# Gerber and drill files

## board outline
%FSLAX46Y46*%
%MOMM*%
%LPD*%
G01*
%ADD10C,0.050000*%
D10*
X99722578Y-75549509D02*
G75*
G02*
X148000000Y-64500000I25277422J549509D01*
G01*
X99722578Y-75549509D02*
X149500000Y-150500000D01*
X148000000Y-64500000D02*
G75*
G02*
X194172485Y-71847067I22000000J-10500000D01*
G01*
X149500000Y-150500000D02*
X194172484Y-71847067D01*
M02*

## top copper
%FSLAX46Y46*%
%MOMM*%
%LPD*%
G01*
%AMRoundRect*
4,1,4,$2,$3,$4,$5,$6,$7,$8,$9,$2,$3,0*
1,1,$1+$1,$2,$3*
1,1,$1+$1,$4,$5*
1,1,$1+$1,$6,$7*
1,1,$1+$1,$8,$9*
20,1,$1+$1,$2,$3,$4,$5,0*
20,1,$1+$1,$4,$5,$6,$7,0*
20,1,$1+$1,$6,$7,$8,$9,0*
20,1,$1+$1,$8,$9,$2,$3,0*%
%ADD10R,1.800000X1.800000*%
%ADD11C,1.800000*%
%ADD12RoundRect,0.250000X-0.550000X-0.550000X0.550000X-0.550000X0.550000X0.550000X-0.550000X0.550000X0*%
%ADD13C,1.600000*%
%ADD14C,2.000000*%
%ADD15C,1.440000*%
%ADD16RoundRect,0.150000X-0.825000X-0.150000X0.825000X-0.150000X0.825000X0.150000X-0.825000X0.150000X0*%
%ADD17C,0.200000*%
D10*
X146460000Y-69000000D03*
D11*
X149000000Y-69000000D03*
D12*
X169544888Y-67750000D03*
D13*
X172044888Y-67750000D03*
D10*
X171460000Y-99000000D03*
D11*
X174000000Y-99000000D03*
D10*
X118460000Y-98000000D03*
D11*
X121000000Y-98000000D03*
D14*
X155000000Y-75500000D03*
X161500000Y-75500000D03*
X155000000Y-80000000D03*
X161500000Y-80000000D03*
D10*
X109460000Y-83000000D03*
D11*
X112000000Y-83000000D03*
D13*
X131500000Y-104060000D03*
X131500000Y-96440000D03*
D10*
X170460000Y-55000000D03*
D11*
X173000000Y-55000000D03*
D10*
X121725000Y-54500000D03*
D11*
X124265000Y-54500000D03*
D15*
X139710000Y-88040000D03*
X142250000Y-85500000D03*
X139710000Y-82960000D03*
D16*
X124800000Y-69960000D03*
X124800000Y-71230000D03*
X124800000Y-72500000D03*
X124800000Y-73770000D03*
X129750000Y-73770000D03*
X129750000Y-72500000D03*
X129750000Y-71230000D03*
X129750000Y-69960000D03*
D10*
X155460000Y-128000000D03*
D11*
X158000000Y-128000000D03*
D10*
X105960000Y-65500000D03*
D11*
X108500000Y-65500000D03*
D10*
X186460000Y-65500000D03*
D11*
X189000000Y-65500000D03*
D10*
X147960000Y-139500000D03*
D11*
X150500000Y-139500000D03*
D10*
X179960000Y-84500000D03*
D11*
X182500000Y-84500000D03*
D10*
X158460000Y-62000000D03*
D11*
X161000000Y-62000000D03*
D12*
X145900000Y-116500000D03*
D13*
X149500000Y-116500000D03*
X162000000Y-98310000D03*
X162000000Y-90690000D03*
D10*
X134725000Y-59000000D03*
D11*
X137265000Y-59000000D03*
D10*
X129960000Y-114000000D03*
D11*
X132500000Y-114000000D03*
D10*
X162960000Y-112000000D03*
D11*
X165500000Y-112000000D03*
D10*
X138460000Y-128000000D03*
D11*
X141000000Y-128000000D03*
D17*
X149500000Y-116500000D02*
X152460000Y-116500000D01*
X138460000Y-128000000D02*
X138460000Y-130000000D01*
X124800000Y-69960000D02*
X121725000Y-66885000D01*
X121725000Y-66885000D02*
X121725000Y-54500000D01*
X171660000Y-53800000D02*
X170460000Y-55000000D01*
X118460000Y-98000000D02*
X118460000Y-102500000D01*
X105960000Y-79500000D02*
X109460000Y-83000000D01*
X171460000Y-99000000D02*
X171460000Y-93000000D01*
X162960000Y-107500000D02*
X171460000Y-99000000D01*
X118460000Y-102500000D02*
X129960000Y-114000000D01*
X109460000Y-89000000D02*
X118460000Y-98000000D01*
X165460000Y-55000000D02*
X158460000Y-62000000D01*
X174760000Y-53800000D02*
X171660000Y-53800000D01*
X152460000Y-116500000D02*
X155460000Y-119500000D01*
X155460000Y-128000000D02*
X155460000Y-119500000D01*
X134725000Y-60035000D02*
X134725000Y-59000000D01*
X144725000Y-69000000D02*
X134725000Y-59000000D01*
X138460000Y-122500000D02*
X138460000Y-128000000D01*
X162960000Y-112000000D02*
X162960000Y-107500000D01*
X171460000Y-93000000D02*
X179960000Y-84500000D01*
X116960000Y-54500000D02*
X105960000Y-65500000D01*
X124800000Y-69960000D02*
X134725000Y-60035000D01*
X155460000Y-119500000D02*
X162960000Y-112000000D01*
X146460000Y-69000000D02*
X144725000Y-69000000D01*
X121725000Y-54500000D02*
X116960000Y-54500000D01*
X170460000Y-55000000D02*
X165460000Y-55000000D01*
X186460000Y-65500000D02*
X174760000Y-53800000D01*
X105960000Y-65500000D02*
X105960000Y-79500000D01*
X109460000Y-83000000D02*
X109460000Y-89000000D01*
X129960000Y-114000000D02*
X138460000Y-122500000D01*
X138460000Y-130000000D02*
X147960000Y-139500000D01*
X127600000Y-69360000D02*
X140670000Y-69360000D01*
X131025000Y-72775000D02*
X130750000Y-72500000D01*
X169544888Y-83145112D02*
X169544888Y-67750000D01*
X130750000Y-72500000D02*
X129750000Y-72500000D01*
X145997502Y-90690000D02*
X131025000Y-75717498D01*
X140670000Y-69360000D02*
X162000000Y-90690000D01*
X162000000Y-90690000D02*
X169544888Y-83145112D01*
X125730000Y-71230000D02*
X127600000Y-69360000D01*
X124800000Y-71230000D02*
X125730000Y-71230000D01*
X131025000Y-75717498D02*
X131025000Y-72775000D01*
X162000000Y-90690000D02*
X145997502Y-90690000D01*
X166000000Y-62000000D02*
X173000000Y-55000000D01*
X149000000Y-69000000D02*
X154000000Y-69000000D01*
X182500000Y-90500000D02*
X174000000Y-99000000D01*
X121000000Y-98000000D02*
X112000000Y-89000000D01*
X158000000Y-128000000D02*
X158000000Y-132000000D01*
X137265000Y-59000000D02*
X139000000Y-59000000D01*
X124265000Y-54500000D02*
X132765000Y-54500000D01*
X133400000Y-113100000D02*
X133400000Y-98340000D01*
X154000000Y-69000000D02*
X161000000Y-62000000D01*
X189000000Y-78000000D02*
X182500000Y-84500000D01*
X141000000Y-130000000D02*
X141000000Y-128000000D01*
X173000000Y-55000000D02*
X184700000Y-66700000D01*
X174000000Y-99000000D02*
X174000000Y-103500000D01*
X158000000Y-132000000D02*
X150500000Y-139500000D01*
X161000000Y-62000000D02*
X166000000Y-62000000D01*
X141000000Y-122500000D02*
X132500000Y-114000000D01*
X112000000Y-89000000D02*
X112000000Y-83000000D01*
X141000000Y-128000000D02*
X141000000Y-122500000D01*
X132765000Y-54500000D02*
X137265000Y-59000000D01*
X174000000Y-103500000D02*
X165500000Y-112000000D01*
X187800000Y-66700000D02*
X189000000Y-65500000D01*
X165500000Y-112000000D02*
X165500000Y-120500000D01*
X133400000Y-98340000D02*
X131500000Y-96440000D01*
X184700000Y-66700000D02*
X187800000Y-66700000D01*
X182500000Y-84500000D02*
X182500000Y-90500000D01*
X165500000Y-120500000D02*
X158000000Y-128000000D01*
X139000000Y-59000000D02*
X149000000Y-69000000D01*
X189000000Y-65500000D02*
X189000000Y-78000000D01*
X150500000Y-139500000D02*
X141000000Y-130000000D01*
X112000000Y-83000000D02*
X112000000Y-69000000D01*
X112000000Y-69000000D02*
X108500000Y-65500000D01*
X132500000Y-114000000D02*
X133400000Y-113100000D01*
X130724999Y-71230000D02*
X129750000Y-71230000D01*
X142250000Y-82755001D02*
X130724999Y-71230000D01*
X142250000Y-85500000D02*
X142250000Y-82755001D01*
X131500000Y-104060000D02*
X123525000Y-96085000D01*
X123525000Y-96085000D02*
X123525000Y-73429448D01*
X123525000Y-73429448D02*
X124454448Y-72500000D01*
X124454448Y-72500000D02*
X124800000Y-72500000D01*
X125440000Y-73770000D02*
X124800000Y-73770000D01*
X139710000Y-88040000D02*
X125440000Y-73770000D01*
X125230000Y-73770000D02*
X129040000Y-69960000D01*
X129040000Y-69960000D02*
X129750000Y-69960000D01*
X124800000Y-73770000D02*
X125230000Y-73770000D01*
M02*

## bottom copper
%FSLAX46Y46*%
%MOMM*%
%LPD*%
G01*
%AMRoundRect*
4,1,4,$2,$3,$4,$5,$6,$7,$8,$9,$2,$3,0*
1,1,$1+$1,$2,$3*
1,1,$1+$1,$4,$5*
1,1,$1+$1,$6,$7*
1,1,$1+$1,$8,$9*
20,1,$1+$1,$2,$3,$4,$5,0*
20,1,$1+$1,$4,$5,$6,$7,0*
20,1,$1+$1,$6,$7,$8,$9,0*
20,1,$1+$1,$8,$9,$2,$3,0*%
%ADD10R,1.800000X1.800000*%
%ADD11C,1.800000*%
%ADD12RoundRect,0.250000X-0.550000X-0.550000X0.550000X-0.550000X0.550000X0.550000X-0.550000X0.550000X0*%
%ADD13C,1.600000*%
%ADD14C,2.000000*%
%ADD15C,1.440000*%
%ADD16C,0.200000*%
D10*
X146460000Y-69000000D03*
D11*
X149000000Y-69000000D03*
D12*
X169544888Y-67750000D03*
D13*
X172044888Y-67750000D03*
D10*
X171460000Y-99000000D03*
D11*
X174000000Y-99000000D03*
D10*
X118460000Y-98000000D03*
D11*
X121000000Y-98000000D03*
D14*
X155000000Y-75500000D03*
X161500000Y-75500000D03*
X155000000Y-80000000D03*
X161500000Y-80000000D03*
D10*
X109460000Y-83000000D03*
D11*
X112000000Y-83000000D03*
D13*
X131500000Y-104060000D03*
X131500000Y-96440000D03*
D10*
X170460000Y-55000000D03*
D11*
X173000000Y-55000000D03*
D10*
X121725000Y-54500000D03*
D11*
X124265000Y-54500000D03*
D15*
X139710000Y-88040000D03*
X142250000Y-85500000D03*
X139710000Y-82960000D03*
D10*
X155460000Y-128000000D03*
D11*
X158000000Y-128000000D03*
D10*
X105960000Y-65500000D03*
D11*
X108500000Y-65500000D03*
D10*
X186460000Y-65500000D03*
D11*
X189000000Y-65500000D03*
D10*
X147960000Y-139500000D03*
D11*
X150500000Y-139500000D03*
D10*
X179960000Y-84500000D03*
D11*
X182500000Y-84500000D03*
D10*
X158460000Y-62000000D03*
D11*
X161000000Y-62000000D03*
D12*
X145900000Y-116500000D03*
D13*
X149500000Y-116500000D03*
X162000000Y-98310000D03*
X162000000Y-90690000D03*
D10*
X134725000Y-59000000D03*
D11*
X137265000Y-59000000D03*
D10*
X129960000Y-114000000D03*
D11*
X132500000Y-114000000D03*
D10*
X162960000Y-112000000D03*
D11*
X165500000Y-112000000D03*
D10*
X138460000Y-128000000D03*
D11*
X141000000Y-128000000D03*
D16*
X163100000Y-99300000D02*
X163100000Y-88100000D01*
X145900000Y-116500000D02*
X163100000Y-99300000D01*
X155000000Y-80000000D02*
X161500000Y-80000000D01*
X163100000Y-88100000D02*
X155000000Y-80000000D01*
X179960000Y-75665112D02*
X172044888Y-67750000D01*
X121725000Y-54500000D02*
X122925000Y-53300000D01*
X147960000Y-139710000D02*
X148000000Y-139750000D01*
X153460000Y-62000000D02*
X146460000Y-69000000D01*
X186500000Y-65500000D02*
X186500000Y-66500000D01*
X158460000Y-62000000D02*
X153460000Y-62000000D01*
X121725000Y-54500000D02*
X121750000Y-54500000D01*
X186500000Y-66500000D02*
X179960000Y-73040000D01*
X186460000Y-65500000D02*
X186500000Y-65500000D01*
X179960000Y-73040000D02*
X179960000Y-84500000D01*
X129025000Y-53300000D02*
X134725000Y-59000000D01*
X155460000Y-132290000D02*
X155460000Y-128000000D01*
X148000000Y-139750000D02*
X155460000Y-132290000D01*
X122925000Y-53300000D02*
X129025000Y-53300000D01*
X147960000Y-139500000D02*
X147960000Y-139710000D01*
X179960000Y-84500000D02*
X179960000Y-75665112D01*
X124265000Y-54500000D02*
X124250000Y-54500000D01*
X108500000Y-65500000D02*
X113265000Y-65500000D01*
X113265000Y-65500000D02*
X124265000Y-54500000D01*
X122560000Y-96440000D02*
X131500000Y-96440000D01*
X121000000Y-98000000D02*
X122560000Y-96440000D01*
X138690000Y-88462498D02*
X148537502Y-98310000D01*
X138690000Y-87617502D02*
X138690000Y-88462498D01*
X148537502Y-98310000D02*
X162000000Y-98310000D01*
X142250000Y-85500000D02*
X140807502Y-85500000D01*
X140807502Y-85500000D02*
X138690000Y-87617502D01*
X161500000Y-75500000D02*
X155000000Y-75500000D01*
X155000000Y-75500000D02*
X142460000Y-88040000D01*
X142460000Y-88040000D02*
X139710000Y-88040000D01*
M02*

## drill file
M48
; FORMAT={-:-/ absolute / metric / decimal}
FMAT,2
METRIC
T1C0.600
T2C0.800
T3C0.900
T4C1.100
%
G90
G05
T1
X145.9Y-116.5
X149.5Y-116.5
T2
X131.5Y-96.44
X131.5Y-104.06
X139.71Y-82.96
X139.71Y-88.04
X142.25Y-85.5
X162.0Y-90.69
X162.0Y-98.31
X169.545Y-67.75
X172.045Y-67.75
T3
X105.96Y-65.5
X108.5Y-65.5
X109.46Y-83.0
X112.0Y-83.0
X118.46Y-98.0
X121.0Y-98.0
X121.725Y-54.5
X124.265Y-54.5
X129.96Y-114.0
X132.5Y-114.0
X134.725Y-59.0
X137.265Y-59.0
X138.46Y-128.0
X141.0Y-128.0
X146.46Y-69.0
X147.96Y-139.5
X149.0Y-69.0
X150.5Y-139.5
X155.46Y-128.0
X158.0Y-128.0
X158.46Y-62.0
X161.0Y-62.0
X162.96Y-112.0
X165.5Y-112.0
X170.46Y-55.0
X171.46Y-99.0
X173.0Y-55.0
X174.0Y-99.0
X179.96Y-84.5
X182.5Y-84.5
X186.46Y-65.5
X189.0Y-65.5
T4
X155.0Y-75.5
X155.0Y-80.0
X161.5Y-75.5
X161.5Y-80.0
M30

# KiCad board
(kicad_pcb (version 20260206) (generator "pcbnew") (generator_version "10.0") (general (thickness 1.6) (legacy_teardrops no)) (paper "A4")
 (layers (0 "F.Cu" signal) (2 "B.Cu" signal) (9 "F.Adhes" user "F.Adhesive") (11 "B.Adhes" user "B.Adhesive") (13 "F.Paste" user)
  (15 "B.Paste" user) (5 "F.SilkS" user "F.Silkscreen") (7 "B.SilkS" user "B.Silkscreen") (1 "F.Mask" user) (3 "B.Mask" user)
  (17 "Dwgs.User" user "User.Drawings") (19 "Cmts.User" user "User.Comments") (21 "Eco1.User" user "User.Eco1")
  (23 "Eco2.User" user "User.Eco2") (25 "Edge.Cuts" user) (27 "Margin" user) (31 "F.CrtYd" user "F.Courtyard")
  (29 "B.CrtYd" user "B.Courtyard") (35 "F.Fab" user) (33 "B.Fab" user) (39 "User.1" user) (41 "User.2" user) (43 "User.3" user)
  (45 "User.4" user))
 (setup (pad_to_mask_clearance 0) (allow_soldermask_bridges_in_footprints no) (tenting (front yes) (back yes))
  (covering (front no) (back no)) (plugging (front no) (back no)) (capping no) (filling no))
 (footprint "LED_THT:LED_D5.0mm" (layer "F.Cu") (at 146.46 69)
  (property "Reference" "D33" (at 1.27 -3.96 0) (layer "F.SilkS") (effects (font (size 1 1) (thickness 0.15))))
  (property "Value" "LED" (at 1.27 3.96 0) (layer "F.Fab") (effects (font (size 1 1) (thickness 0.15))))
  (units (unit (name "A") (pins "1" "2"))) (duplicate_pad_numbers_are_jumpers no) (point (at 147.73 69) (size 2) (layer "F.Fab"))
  (pad "1" thru_hole rect (at 0 0) (size 1.8 1.8) (drill 0.9) (layers "*.Cu" "*.Mask") (remove_unused_layers no) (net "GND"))
  (pad "2" thru_hole circle (at 2.54 0) (size 1.8 1.8) (drill 0.9) (layers "*.Cu" "*.Mask") (remove_unused_layers no) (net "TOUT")))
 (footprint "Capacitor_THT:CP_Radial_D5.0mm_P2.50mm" (layer "F.Cu") (at 169.544888 67.75)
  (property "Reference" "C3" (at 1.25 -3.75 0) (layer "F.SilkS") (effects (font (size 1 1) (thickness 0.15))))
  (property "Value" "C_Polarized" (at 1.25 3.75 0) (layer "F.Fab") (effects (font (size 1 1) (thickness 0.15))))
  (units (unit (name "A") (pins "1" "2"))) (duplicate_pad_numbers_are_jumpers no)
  (pad "1" thru_hole roundrect (at 0 0) (size 1.6 1.6) (drill 0.8) (layers "*.Cu" "*.Mask") (remove_unused_layers no)
   (roundrect_rratio 0.15625) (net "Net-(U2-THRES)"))
  (pad "2" thru_hole circle (at 2.5 0) (size 1.6 1.6) (drill 0.8) (layers "*.Cu" "*.Mask") (remove_unused_layers no) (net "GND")))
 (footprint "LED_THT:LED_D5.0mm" (layer "F.Cu") (at 171.46 99)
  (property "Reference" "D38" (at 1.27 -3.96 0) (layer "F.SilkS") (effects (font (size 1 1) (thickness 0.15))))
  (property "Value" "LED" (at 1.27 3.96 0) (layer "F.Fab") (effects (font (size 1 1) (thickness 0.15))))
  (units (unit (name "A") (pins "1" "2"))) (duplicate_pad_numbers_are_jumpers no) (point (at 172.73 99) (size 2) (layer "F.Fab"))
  (pad "1" thru_hole rect (at 0 0) (size 1.8 1.8) (drill 0.9) (layers "*.Cu" "*.Mask") (remove_unused_layers no) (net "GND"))
  (pad "2" thru_hole circle (at 2.54 0) (size 1.8 1.8) (drill 0.9) (layers "*.Cu" "*.Mask") (remove_unused_layers no) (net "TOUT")))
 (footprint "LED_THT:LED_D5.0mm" (layer "F.Cu") (at 118.46 98)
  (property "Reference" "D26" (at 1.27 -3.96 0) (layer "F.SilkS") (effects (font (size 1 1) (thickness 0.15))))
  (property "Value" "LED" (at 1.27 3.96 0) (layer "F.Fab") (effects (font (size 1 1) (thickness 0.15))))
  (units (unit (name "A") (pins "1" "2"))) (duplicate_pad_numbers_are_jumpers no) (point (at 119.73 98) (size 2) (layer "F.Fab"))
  (pad "1" thru_hole rect (at 0 0) (size 1.8 1.8) (drill 0.9) (layers "*.Cu" "*.Mask") (remove_unused_layers no) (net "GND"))
  (pad "2" thru_hole circle (at 2.54 0) (size 1.8 1.8) (drill 0.9) (layers "*.Cu" "*.Mask") (remove_unused_layers no) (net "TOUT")))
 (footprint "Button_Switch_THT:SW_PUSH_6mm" (layer "F.Cu") (at 155 75.5)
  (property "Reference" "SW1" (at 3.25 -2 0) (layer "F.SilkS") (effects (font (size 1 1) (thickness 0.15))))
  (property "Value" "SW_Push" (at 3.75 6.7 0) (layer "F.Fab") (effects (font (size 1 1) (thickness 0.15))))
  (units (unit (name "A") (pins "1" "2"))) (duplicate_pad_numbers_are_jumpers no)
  (pad "1" thru_hole circle (at 0 0 90) (size 2 2) (drill 1.1) (layers "*.Cu" "*.Mask") (remove_unused_layers no) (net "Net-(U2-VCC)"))
  (pad "1" thru_hole circle (at 6.5 0 90) (size 2 2) (drill 1.1) (layers "*.Cu" "*.Mask") (remove_unused_layers no) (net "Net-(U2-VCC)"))
  (pad "2" thru_hole circle (at 0 4.5 90) (size 2 2) (drill 1.1) (layers "*.Cu" "*.Mask") (remove_unused_layers no) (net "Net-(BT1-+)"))
  (pad "2" thru_hole circle (at 6.5 4.5 90) (size 2 2) (drill 1.1) (layers "*.Cu" "*.Mask") (remove_unused_layers no) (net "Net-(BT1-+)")))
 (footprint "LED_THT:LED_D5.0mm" (layer "F.Cu") (at 109.46 83)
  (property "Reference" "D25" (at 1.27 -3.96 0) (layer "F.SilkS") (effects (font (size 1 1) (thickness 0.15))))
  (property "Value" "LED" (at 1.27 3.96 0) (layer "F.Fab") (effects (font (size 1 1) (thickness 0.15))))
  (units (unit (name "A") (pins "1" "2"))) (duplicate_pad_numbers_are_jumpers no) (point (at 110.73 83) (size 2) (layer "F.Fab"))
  (pad "1" thru_hole rect (at 0 0) (size 1.8 1.8) (drill 0.9) (layers "*.Cu" "*.Mask") (remove_unused_layers no) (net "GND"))
  (pad "2" thru_hole circle (at 2.54 0) (size 1.8 1.8) (drill 0.9) (layers "*.Cu" "*.Mask") (remove_unused_layers no) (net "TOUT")))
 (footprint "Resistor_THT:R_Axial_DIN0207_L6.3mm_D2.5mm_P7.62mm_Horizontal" (layer "F.Cu") (at 131.5 104.06 90)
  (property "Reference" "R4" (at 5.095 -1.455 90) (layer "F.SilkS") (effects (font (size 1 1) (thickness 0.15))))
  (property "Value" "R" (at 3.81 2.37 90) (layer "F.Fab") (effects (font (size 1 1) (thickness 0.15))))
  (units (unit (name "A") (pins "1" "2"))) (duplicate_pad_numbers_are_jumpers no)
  (pad "1" thru_hole circle (at 0 0 90) (size 1.6 1.6) (drill 0.8) (layers "*.Cu" "*.Mask") (remove_unused_layers no) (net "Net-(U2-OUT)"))
  (pad "2" thru_hole circle (at 7.62 0 90) (size 1.6 1.6) (drill 0.8) (layers "*.Cu" "*.Mask") (remove_unused_layers no) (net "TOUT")))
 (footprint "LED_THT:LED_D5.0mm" (layer "F.Cu") (at 170.46 55)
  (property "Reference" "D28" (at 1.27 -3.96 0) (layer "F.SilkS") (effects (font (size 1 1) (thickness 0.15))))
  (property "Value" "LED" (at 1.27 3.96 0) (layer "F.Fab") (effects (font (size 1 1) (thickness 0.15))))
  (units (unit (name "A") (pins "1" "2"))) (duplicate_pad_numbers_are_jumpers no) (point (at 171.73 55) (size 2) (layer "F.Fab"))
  (pad "1" thru_hole rect (at 0 0) (size 1.8 1.8) (drill 0.9) (layers "*.Cu" "*.Mask") (remove_unused_layers no) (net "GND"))
  (pad "2" thru_hole circle (at 2.54 0) (size 1.8 1.8) (drill 0.9) (layers "*.Cu" "*.Mask") (remove_unused_layers no) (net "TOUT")))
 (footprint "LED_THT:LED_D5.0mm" (layer "F.Cu") (at 121.725 54.5)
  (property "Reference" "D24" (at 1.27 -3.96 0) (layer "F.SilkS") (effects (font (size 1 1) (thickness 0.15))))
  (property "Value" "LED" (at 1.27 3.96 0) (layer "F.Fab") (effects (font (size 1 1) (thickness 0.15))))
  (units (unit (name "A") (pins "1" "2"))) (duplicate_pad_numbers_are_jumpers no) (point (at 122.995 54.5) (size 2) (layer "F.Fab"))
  (pad "1" thru_hole rect (at 0 0) (size 1.8 1.8) (drill 0.9) (layers "*.Cu" "*.Mask") (remove_unused_layers no) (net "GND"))
  (pad "2" thru_hole circle (at 2.54 0) (size 1.8 1.8) (drill 0.9) (layers "*.Cu" "*.Mask") (remove_unused_layers no) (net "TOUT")))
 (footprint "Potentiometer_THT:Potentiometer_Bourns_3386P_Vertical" (layer "F.Cu") (at 139.71 88.04)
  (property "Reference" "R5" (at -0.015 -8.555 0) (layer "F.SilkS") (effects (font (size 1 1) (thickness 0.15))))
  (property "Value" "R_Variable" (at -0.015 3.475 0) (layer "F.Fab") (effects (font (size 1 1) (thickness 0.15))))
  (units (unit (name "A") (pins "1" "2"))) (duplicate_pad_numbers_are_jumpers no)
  (pad "1" thru_hole circle (at 0 0) (size 1.44 1.44) (drill 0.8) (layers "*.Cu" "*.Mask") (remove_unused_layers no) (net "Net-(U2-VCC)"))
  (pad "2" thru_hole circle (at 2.54 -2.54) (size 1.44 1.44) (drill 0.8) (layers "*.Cu" "*.Mask") (remove_unused_layers no)
   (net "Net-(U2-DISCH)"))
  (pad "3" thru_hole circle (at 0 -5.08) (size 1.44 1.44) (drill 0.8) (layers "*.Cu" "*.Mask") (remove_unused_layers no)))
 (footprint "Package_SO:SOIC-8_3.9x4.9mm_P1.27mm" (layer "F.Cu") (at 127.275 71.865)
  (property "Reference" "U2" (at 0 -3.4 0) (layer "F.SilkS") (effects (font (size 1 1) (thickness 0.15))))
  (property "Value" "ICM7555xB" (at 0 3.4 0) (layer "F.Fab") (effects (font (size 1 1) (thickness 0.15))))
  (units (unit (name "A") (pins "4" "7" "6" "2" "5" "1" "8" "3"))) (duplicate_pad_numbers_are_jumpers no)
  (pad "1" smd roundrect (at -2.475 -1.905) (size 1.95 0.6) (layers "F.Cu" "F.Mask" "F.Paste") (roundrect_rratio 0.25) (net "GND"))
  (pad "2" smd roundrect (at -2.475 -0.635) (size 1.95 0.6) (layers "F.Cu" "F.Mask" "F.Paste") (roundrect_rratio 0.25)
   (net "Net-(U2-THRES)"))
  (pad "3" smd roundrect (at -2.475 0.635) (size 1.95 0.6) (layers "F.Cu" "F.Mask" "F.Paste") (roundrect_rratio 0.25) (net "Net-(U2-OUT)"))
  (pad "4" smd roundrect (at -2.475 1.905) (size 1.95 0.6) (layers "F.Cu" "F.Mask" "F.Paste") (roundrect_rratio 0.25) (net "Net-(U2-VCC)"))
  (pad "5" smd roundrect (at 2.475 1.905) (size 1.95 0.6) (layers "F.Cu" "F.Mask" "F.Paste") (roundrect_rratio 0.25)
   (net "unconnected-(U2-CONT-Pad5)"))
  (pad "6" smd roundrect (at 2.475 0.635) (size 1.95 0.6) (layers "F.Cu" "F.Mask" "F.Paste") (roundrect_rratio 0.25) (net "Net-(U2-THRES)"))
  (pad "7" smd roundrect (at 2.475 -0.635) (size 1.95 0.6) (layers "F.Cu" "F.Mask" "F.Paste") (roundrect_rratio 0.25) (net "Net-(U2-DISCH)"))
  (pad "8" smd roundrect (at 2.475 -1.905) (size 1.95 0.6) (layers "F.Cu" "F.Mask" "F.Paste") (roundrect_rratio 0.25) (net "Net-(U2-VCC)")))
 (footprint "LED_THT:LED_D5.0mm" (layer "F.Cu") (at 155.46 128)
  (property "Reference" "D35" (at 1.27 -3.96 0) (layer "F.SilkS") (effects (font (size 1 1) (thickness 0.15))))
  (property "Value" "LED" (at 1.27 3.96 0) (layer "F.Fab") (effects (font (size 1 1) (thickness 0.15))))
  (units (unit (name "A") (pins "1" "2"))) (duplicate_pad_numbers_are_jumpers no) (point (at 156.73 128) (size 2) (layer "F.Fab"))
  (pad "1" thru_hole rect (at 0 0) (size 1.8 1.8) (drill 0.9) (layers "*.Cu" "*.Mask") (remove_unused_layers no) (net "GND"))
  (pad "2" thru_hole circle (at 2.54 0) (size 1.8 1.8) (drill 0.9) (layers "*.Cu" "*.Mask") (remove_unused_layers no) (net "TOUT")))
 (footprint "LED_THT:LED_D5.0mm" (layer "F.Cu") (at 105.96 65.5)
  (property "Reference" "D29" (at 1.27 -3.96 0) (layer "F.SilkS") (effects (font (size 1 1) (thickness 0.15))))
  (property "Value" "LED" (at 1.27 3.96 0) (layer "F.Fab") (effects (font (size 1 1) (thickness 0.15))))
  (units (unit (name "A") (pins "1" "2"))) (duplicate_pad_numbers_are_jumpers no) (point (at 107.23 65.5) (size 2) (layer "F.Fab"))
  (pad "1" thru_hole rect (at 0 0) (size 1.8 1.8) (drill 0.9) (layers "*.Cu" "*.Mask") (remove_unused_layers no) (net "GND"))
  (pad "2" thru_hole circle (at 2.54 0) (size 1.8 1.8) (drill 0.9) (layers "*.Cu" "*.Mask") (remove_unused_layers no) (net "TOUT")))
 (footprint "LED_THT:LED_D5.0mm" (layer "F.Cu") (at 186.46 65.5)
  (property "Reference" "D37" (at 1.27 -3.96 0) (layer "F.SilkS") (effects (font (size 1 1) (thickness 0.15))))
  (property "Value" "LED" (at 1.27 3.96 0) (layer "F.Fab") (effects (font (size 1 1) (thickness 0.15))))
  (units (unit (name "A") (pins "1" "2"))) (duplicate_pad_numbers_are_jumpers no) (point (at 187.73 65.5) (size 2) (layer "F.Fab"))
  (pad "1" thru_hole rect (at 0 0) (size 1.8 1.8) (drill 0.9) (layers "*.Cu" "*.Mask") (remove_unused_layers no) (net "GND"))
  (pad "2" thru_hole circle (at 2.54 0) (size 1.8 1.8) (drill 0.9) (layers "*.Cu" "*.Mask") (remove_unused_layers no) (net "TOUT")))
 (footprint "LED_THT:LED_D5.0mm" (layer "F.Cu") (at 147.96 139.5)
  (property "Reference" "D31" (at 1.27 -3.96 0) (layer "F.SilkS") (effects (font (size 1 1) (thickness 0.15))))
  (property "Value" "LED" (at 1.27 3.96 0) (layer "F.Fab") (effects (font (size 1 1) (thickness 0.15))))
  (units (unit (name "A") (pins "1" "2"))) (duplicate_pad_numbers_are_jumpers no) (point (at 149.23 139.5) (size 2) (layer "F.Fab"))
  (pad "1" thru_hole rect (at 0 0) (size 1.8 1.8) (drill 0.9) (layers "*.Cu" "*.Mask") (remove_unused_layers no) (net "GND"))
  (pad "2" thru_hole circle (at 2.54 0) (size 1.8 1.8) (drill 0.9) (layers "*.Cu" "*.Mask") (remove_unused_layers no) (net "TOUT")))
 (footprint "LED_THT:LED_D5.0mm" (layer "F.Cu") (at 179.96 84.5)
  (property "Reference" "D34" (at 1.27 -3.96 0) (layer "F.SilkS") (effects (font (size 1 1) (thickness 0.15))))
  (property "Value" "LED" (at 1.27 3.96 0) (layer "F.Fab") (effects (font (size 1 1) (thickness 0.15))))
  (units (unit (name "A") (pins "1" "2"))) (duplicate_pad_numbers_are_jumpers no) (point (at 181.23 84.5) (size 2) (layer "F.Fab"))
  (pad "1" thru_hole rect (at 0 0) (size 1.8 1.8) (drill 0.9) (layers "*.Cu" "*.Mask") (remove_unused_layers no) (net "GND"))
  (pad "2" thru_hole circle (at 2.54 0) (size 1.8 1.8) (drill 0.9) (layers "*.Cu" "*.Mask") (remove_unused_layers no) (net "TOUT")))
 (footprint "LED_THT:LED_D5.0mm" (layer "F.Cu") (at 158.46 62)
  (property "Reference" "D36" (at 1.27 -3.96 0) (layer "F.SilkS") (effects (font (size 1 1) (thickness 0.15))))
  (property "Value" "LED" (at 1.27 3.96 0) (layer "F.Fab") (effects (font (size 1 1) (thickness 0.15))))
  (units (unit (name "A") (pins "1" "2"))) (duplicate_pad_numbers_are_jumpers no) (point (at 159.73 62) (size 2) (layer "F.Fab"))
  (pad "1" thru_hole rect (at 0 0) (size 1.8 1.8) (drill 0.9) (layers "*.Cu" "*.Mask") (remove_unused_layers no) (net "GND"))
  (pad "2" thru_hole circle (at 2.54 0) (size 1.8 1.8) (drill 0.9) (layers "*.Cu" "*.Mask") (remove_unused_layers no) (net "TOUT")))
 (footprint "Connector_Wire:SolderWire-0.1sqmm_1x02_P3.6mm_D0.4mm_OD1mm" (layer "F.Cu") (at 145.9 116.5)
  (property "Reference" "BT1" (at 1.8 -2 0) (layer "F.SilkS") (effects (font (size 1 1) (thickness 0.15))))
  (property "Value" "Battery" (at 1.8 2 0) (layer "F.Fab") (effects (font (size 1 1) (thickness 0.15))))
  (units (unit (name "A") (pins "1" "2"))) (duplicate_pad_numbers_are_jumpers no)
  (pad "1" thru_hole roundrect (at 0 0) (size 1.6 1.6) (drill 0.6) (layers "*.Cu" "*.Mask") (remove_unused_layers no)
   (roundrect_rratio 0.15625) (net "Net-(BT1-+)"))
  (pad "2" thru_hole circle (at 3.6 0) (size 1.6 1.6) (drill 0.6) (layers "*.Cu" "*.Mask") (remove_unused_layers no) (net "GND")))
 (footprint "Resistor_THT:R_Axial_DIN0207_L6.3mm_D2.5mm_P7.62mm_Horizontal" (layer "F.Cu") (at 162 98.31 90)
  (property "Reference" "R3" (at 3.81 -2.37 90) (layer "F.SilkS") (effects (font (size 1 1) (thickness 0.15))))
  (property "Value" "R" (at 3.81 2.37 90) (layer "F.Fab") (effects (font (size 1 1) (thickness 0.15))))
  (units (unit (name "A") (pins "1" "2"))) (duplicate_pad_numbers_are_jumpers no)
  (pad "1" thru_hole circle (at 0 0 90) (size 1.6 1.6) (drill 0.8) (layers "*.Cu" "*.Mask") (remove_unused_layers no) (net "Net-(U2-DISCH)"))
  (pad "2" thru_hole circle (at 7.62 0 90) (size 1.6 1.6) (drill 0.8) (layers "*.Cu" "*.Mask") (remove_unused_layers no)
   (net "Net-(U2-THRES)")))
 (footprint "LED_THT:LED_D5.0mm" (layer "F.Cu") (at 134.725 59)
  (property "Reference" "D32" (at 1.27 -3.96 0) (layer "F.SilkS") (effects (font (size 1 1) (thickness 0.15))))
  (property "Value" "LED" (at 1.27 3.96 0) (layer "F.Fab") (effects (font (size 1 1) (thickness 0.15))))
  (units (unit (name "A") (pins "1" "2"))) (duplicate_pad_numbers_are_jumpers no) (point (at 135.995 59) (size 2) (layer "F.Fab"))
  (pad "1" thru_hole rect (at 0 0) (size 1.8 1.8) (drill 0.9) (layers "*.Cu" "*.Mask") (remove_unused_layers no) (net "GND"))
  (pad "2" thru_hole circle (at 2.54 0) (size 1.8 1.8) (drill 0.9) (layers "*.Cu" "*.Mask") (remove_unused_layers no) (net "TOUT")))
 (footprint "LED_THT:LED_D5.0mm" (layer "F.Cu") (at 129.96 114)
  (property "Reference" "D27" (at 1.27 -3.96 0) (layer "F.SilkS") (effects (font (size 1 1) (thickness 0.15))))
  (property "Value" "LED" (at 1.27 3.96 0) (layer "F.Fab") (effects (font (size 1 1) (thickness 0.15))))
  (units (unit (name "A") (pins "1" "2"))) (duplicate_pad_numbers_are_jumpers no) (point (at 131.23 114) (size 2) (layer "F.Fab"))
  (pad "1" thru_hole rect (at 0 0) (size 1.8 1.8) (drill 0.9) (layers "*.Cu" "*.Mask") (remove_unused_layers no) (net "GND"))
  (pad "2" thru_hole circle (at 2.54 0) (size 1.8 1.8) (drill 0.9) (layers "*.Cu" "*.Mask") (remove_unused_layers no) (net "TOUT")))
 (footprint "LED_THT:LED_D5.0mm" (layer "F.Cu") (at 162.96 112)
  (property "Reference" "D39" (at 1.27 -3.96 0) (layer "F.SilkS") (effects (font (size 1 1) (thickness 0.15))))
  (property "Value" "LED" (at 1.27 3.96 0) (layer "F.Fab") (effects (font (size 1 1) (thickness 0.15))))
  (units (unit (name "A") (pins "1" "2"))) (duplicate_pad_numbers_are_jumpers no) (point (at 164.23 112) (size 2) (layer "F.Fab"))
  (pad "1" thru_hole rect (at 0 0) (size 1.8 1.8) (drill 0.9) (layers "*.Cu" "*.Mask") (remove_unused_layers no) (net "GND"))
  (pad "2" thru_hole circle (at 2.54 0) (size 1.8 1.8) (drill 0.9) (layers "*.Cu" "*.Mask") (remove_unused_layers no) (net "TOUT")))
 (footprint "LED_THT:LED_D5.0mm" (layer "F.Cu") (at 138.46 128)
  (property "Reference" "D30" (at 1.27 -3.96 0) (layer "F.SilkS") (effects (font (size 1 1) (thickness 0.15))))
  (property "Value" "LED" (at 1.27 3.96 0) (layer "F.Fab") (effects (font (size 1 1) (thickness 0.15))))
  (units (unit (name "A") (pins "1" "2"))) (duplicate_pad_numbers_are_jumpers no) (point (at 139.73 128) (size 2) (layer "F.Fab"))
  (pad "1" thru_hole rect (at 0 0) (size 1.8 1.8) (drill 0.9) (layers "*.Cu" "*.Mask") (remove_unused_layers no) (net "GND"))
  (pad "2" thru_hole circle (at 2.54 0) (size 1.8 1.8) (drill 0.9) (layers "*.Cu" "*.Mask") (remove_unused_layers no) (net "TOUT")))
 (gr_arc (start 99.722578 75.549509) (mid 119.359116 50.353896) (end 148 64.5) (stroke (width 0.05) (type default)) (layer "Edge.Cuts"))
 (gr_line (start 99.722578 75.549509) (end 149.5 150.5) (stroke (width 0.05) (type default)) (layer "Edge.Cuts"))
 (gr_arc (start 148 64.5) (mid 173.830766 50.925631) (end 194.172484 71.847067) (stroke (width 0.05) (type default)) (layer "Edge.Cuts"))
 (gr_line (start 149.5 150.5) (end 194.172484 71.847067) (stroke (width 0.05) (type default)) (layer "Edge.Cuts"))
 (segment (start 163.1 99.3) (end 163.1 88.1) (width 0.2) (layer "B.Cu") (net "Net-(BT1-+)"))
 (segment (start 145.9 116.5) (end 163.1 99.3) (width 0.2) (layer "B.Cu") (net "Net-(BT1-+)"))
 (segment (start 155 80) (end 161.5 80) (width 0.2) (layer "B.Cu") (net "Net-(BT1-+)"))
 (segment (start 163.1 88.1) (end 155 80) (width 0.2) (layer "B.Cu") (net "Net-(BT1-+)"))
 (segment (start 149.5 116.5) (end 152.46 116.5) (width 0.2) (layer "F.Cu") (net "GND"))
 (segment (start 138.46 128) (end 138.46 130) (width 0.2) (layer "F.Cu") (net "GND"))
 (segment (start 124.8 69.96) (end 121.725 66.885) (width 0.2) (layer "F.Cu") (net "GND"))
 (segment (start 121.725 66.885) (end 121.725 54.5) (width 0.2) (layer "F.Cu") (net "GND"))
 (segment (start 171.66 53.8) (end 170.46 55) (width 0.2) (layer "F.Cu") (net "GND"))
 (segment (start 118.46 98) (end 118.46 102.5) (width 0.2) (layer "F.Cu") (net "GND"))
 (segment (start 105.96 79.5) (end 109.46 83) (width 0.2) (layer "F.Cu") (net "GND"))
 (segment (start 171.46 99) (end 171.46 93) (width 0.2) (layer "F.Cu") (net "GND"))
 (segment (start 162.96 107.5) (end 171.46 99) (width 0.2) (layer "F.Cu") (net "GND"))
 (segment (start 118.46 102.5) (end 129.96 114) (width 0.2) (layer "F.Cu") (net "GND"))
 (segment (start 109.46 89) (end 118.46 98) (width 0.2) (layer "F.Cu") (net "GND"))
 (segment (start 165.46 55) (end 158.46 62) (width 0.2) (layer "F.Cu") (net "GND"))
 (segment (start 174.76 53.8) (end 171.66 53.8) (width 0.2) (layer "F.Cu") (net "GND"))
 (segment (start 152.46 116.5) (end 155.46 119.5) (width 0.2) (layer "F.Cu") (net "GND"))
 (segment (start 155.46 128) (end 155.46 119.5) (width 0.2) (layer "F.Cu") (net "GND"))
 (segment (start 134.725 60.035) (end 134.725 59) (width 0.2) (layer "F.Cu") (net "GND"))
 (segment (start 144.725 69) (end 134.725 59) (width 0.2) (layer "F.Cu") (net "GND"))
 (segment (start 138.46 122.5) (end 138.46 128) (width 0.2) (layer "F.Cu") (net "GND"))
 (segment (start 162.96 112) (end 162.96 107.5) (width 0.2) (layer "F.Cu") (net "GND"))
 (segment (start 171.46 93) (end 179.96 84.5) (width 0.2) (layer "F.Cu") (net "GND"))
 (segment (start 116.96 54.5) (end 105.96 65.5) (width 0.2) (layer "F.Cu") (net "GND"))
 (segment (start 124.8 69.96) (end 134.725 60.035) (width 0.2) (layer "F.Cu") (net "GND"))
 (segment (start 155.46 119.5) (end 162.96 112) (width 0.2) (layer "F.Cu") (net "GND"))
 (segment (start 146.46 69) (end 144.725 69) (width 0.2) (layer "F.Cu") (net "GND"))
 (segment (start 121.725 54.5) (end 116.96 54.5) (width 0.2) (layer "F.Cu") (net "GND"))
 (segment (start 170.46 55) (end 165.46 55) (width 0.2) (layer "F.Cu") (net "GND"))
 (segment (start 186.46 65.5) (end 174.76 53.8) (width 0.2) (layer "F.Cu") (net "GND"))
 (segment (start 105.96 65.5) (end 105.96 79.5) (width 0.2) (layer "F.Cu") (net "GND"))
 (segment (start 109.46 83) (end 109.46 89) (width 0.2) (layer "F.Cu") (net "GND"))
 (segment (start 129.96 114) (end 138.46 122.5) (width 0.2) (layer "F.Cu") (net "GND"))
 (segment (start 138.46 130) (end 147.96 139.5) (width 0.2) (layer "F.Cu") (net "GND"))
 (segment (start 179.96 75.665112) (end 172.044888 67.75) (width 0.2) (layer "B.Cu") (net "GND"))
 (segment (start 121.725 54.5) (end 122.925 53.3) (width 0.2) (layer "B.Cu") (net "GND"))
 (segment (start 147.96 139.71) (end 148 139.75) (width 0.2) (layer "B.Cu") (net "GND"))
 (segment (start 153.46 62) (end 146.46 69) (width 0.2) (layer "B.Cu") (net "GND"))
 (segment (start 186.5 65.5) (end 186.5 66.5) (width 0.2) (layer "B.Cu") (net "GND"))
 (segment (start 158.46 62) (end 153.46 62) (width 0.2) (layer "B.Cu") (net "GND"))
 (segment (start 121.725 54.5) (end 121.75 54.5) (width 0.2) (layer "B.Cu") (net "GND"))
 (segment (start 186.5 66.5) (end 179.96 73.04) (width 0.2) (layer "B.Cu") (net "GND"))
 (segment (start 186.46 65.5) (end 186.5 65.5) (width 0.2) (layer "B.Cu") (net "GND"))
 (segment (start 179.96 73.04) (end 179.96 84.5) (width 0.2) (layer "B.Cu") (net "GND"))
 (segment (start 129.025 53.3) (end 134.725 59) (width 0.2) (layer "B.Cu") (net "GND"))
 (segment (start 155.46 132.29) (end 155.46 128) (width 0.2) (layer "B.Cu") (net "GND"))
 (segment (start 148 139.75) (end 155.46 132.29) (width 0.2) (layer "B.Cu") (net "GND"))
 (segment (start 122.925 53.3) (end 129.025 53.3) (width 0.2) (layer "B.Cu") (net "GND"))
 (segment (start 147.96 139.5) (end 147.96 139.71) (width 0.2) (layer "B.Cu") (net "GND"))
 (segment (start 179.96 84.5) (end 179.96 75.665112) (width 0.2) (layer "B.Cu") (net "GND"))
 (segment (start 127.6 69.36) (end 140.67 69.36) (width 0.2) (layer "F.Cu") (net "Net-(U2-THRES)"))
 (segment (start 131.025 72.775) (end 130.75 72.5) (width 0.2) (layer "F.Cu") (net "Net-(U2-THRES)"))
 (segment (start 169.544888 83.145112) (end 169.544888 67.75) (width 0.2) (layer "F.Cu") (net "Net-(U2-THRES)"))
 (segment (start 130.75 72.5) (end 129.75 72.5) (width 0.2) (layer "F.Cu") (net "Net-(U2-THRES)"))
 (segment (start 145.997502 90.69) (end 131.025 75.717498) (width 0.2) (layer "F.Cu") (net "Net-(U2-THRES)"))
 (segment (start 140.67 69.36) (end 162 90.69) (width 0.2) (layer "F.Cu") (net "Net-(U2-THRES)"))
 (segment (start 162 90.69) (end 169.544888 83.145112) (width 0.2) (layer "F.Cu") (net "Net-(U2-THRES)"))
 (segment (start 125.73 71.23) (end 127.6 69.36) (width 0.2) (layer "F.Cu") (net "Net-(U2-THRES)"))
 (segment (start 124.8 71.23) (end 125.73 71.23) (width 0.2) (layer "F.Cu") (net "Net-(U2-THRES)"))
 (segment (start 131.025 75.717498) (end 131.025 72.775) (width 0.2) (layer "F.Cu") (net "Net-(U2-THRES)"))
 (segment (start 162 90.69) (end 145.997502 90.69) (width 0.2) (layer "F.Cu") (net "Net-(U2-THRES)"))
 (segment (start 166 62) (end 173 55) (width 0.2) (layer "F.Cu") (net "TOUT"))
 (segment (start 149 69) (end 154 69) (width 0.2) (layer "F.Cu") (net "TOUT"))
 (segment (start 182.5 90.5) (end 174 99) (width 0.2) (layer "F.Cu") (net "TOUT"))
 (segment (start 121 98) (end 112 89) (width 0.2) (layer "F.Cu") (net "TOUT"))
 (segment (start 158 128) (end 158 132) (width 0.2) (layer "F.Cu") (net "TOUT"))
 (segment (start 137.265 59) (end 139 59) (width 0.2) (layer "F.Cu") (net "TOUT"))
 (segment (start 124.265 54.5) (end 132.765 54.5) (width 0.2) (layer "F.Cu") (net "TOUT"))
 (segment (start 133.4 113.1) (end 133.4 98.34) (width 0.2) (layer "F.Cu") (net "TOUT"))
 (segment (start 154 69) (end 161 62) (width 0.2) (layer "F.Cu") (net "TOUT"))
 (segment (start 189 78) (end 182.5 84.5) (width 0.2) (layer "F.Cu") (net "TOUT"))
 (segment (start 141 130) (end 141 128) (width 0.2) (layer "F.Cu") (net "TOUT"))
 (segment (start 173 55) (end 184.7 66.7) (width 0.2) (layer "F.Cu") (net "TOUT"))
 (segment (start 174 99) (end 174 103.5) (width 0.2) (layer "F.Cu") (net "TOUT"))
 (segment (start 158 132) (end 150.5 139.5) (width 0.2) (layer "F.Cu") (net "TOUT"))
 (segment (start 161 62) (end 166 62) (width 0.2) (layer "F.Cu") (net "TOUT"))
 (segment (start 141 122.5) (end 132.5 114) (width 0.2) (layer "F.Cu") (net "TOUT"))
 (segment (start 112 89) (end 112 83) (width 0.2) (layer "F.Cu") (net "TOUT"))
 (segment (start 141 128) (end 141 122.5) (width 0.2) (layer "F.Cu") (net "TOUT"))
 (segment (start 132.765 54.5) (end 137.265 59) (width 0.2) (layer "F.Cu") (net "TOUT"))
 (segment (start 174 103.5) (end 165.5 112) (width 0.2) (layer "F.Cu") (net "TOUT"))
 (segment (start 187.8 66.7) (end 189 65.5) (width 0.2) (layer "F.Cu") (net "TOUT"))
 (segment (start 165.5 112) (end 165.5 120.5) (width 0.2) (layer "F.Cu") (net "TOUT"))
 (segment (start 133.4 98.34) (end 131.5 96.44) (width 0.2) (layer "F.Cu") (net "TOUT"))
 (segment (start 184.7 66.7) (end 187.8 66.7) (width 0.2) (layer "F.Cu") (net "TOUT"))
 (segment (start 182.5 84.5) (end 182.5 90.5) (width 0.2) (layer "F.Cu") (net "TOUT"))
 (segment (start 165.5 120.5) (end 158 128) (width 0.2) (layer "F.Cu") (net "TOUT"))
 (segment (start 139 59) (end 149 69) (width 0.2) (layer "F.Cu") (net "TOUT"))
 (segment (start 189 65.5) (end 189 78) (width 0.2) (layer "F.Cu") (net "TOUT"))
 (segment (start 150.5 139.5) (end 141 130) (width 0.2) (layer "F.Cu") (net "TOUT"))
 (segment (start 112 83) (end 112 69) (width 0.2) (layer "F.Cu") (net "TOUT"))
 (segment (start 112 69) (end 108.5 65.5) (width 0.2) (layer "F.Cu") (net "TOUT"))
 (segment (start 132.5 114) (end 133.4 113.1) (width 0.2) (layer "F.Cu") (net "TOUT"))
 (segment (start 124.265 54.5) (end 124.25 54.5) (width 0.2) (layer "B.Cu") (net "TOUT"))
 (segment (start 108.5 65.5) (end 113.265 65.5) (width 0.2) (layer "B.Cu") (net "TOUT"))
 (segment (start 113.265 65.5) (end 124.265 54.5) (width 0.2) (layer "B.Cu") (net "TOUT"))
 (segment (start 122.56 96.44) (end 131.5 96.44) (width 0.2) (layer "B.Cu") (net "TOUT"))
 (segment (start 121 98) (end 122.56 96.44) (width 0.2) (layer "B.Cu") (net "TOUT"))
 (segment (start 130.724999 71.23) (end 129.75 71.23) (width 0.2) (layer "F.Cu") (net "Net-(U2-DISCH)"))
 (segment (start 142.25 82.755001) (end 130.724999 71.23) (width 0.2) (layer "F.Cu") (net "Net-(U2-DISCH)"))
 (segment (start 142.25 85.5) (end 142.25 82.755001) (width 0.2) (layer "F.Cu") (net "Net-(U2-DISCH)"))
 (segment (start 138.69 88.462498) (end 148.537502 98.31) (width 0.2) (layer "B.Cu") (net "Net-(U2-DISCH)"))
 (segment (start 138.69 87.617502) (end 138.69 88.462498) (width 0.2) (layer "B.Cu") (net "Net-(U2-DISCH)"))
 (segment (start 148.537502 98.31) (end 162 98.31) (width 0.2) (layer "B.Cu") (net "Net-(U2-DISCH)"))
 (segment (start 142.25 85.5) (end 140.807502 85.5) (width 0.2) (layer "B.Cu") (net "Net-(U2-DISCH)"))
 (segment (start 140.807502 85.5) (end 138.69 87.617502) (width 0.2) (layer "B.Cu") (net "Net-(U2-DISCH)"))
 (segment (start 131.5 104.06) (end 123.525 96.085) (width 0.2) (layer "F.Cu") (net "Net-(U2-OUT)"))
 (segment (start 123.525 96.085) (end 123.525 73.429448) (width 0.2) (layer "F.Cu") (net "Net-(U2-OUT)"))
 (segment (start 123.525 73.429448) (end 124.454448 72.5) (width 0.2) (layer "F.Cu") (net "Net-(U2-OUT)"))
 (segment (start 124.454448 72.5) (end 124.8 72.5) (width 0.2) (layer "F.Cu") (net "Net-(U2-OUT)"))
 (segment (start 125.44 73.77) (end 124.8 73.77) (width 0.2) (layer "F.Cu") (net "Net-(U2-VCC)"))
 (segment (start 139.71 88.04) (end 125.44 73.77) (width 0.2) (layer "F.Cu") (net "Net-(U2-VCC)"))
 (segment (start 125.23 73.77) (end 129.04 69.96) (width 0.2) (layer "F.Cu") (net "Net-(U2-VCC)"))
 (segment (start 129.04 69.96) (end 129.75 69.96) (width 0.2) (layer "F.Cu") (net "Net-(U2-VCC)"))
 (segment (start 124.8 73.77) (end 125.23 73.77) (width 0.2) (layer "F.Cu") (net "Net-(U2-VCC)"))
 (segment (start 161.5 75.5) (end 155 75.5) (width 0.2) (layer "B.Cu") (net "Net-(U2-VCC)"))
 (segment (start 155 75.5) (end 142.46 88.04) (width 0.2) (layer "B.Cu") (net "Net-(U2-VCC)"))
 (segment (start 142.46 88.04) (end 139.71 88.04) (width 0.2) (layer "B.Cu") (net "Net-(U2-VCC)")))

